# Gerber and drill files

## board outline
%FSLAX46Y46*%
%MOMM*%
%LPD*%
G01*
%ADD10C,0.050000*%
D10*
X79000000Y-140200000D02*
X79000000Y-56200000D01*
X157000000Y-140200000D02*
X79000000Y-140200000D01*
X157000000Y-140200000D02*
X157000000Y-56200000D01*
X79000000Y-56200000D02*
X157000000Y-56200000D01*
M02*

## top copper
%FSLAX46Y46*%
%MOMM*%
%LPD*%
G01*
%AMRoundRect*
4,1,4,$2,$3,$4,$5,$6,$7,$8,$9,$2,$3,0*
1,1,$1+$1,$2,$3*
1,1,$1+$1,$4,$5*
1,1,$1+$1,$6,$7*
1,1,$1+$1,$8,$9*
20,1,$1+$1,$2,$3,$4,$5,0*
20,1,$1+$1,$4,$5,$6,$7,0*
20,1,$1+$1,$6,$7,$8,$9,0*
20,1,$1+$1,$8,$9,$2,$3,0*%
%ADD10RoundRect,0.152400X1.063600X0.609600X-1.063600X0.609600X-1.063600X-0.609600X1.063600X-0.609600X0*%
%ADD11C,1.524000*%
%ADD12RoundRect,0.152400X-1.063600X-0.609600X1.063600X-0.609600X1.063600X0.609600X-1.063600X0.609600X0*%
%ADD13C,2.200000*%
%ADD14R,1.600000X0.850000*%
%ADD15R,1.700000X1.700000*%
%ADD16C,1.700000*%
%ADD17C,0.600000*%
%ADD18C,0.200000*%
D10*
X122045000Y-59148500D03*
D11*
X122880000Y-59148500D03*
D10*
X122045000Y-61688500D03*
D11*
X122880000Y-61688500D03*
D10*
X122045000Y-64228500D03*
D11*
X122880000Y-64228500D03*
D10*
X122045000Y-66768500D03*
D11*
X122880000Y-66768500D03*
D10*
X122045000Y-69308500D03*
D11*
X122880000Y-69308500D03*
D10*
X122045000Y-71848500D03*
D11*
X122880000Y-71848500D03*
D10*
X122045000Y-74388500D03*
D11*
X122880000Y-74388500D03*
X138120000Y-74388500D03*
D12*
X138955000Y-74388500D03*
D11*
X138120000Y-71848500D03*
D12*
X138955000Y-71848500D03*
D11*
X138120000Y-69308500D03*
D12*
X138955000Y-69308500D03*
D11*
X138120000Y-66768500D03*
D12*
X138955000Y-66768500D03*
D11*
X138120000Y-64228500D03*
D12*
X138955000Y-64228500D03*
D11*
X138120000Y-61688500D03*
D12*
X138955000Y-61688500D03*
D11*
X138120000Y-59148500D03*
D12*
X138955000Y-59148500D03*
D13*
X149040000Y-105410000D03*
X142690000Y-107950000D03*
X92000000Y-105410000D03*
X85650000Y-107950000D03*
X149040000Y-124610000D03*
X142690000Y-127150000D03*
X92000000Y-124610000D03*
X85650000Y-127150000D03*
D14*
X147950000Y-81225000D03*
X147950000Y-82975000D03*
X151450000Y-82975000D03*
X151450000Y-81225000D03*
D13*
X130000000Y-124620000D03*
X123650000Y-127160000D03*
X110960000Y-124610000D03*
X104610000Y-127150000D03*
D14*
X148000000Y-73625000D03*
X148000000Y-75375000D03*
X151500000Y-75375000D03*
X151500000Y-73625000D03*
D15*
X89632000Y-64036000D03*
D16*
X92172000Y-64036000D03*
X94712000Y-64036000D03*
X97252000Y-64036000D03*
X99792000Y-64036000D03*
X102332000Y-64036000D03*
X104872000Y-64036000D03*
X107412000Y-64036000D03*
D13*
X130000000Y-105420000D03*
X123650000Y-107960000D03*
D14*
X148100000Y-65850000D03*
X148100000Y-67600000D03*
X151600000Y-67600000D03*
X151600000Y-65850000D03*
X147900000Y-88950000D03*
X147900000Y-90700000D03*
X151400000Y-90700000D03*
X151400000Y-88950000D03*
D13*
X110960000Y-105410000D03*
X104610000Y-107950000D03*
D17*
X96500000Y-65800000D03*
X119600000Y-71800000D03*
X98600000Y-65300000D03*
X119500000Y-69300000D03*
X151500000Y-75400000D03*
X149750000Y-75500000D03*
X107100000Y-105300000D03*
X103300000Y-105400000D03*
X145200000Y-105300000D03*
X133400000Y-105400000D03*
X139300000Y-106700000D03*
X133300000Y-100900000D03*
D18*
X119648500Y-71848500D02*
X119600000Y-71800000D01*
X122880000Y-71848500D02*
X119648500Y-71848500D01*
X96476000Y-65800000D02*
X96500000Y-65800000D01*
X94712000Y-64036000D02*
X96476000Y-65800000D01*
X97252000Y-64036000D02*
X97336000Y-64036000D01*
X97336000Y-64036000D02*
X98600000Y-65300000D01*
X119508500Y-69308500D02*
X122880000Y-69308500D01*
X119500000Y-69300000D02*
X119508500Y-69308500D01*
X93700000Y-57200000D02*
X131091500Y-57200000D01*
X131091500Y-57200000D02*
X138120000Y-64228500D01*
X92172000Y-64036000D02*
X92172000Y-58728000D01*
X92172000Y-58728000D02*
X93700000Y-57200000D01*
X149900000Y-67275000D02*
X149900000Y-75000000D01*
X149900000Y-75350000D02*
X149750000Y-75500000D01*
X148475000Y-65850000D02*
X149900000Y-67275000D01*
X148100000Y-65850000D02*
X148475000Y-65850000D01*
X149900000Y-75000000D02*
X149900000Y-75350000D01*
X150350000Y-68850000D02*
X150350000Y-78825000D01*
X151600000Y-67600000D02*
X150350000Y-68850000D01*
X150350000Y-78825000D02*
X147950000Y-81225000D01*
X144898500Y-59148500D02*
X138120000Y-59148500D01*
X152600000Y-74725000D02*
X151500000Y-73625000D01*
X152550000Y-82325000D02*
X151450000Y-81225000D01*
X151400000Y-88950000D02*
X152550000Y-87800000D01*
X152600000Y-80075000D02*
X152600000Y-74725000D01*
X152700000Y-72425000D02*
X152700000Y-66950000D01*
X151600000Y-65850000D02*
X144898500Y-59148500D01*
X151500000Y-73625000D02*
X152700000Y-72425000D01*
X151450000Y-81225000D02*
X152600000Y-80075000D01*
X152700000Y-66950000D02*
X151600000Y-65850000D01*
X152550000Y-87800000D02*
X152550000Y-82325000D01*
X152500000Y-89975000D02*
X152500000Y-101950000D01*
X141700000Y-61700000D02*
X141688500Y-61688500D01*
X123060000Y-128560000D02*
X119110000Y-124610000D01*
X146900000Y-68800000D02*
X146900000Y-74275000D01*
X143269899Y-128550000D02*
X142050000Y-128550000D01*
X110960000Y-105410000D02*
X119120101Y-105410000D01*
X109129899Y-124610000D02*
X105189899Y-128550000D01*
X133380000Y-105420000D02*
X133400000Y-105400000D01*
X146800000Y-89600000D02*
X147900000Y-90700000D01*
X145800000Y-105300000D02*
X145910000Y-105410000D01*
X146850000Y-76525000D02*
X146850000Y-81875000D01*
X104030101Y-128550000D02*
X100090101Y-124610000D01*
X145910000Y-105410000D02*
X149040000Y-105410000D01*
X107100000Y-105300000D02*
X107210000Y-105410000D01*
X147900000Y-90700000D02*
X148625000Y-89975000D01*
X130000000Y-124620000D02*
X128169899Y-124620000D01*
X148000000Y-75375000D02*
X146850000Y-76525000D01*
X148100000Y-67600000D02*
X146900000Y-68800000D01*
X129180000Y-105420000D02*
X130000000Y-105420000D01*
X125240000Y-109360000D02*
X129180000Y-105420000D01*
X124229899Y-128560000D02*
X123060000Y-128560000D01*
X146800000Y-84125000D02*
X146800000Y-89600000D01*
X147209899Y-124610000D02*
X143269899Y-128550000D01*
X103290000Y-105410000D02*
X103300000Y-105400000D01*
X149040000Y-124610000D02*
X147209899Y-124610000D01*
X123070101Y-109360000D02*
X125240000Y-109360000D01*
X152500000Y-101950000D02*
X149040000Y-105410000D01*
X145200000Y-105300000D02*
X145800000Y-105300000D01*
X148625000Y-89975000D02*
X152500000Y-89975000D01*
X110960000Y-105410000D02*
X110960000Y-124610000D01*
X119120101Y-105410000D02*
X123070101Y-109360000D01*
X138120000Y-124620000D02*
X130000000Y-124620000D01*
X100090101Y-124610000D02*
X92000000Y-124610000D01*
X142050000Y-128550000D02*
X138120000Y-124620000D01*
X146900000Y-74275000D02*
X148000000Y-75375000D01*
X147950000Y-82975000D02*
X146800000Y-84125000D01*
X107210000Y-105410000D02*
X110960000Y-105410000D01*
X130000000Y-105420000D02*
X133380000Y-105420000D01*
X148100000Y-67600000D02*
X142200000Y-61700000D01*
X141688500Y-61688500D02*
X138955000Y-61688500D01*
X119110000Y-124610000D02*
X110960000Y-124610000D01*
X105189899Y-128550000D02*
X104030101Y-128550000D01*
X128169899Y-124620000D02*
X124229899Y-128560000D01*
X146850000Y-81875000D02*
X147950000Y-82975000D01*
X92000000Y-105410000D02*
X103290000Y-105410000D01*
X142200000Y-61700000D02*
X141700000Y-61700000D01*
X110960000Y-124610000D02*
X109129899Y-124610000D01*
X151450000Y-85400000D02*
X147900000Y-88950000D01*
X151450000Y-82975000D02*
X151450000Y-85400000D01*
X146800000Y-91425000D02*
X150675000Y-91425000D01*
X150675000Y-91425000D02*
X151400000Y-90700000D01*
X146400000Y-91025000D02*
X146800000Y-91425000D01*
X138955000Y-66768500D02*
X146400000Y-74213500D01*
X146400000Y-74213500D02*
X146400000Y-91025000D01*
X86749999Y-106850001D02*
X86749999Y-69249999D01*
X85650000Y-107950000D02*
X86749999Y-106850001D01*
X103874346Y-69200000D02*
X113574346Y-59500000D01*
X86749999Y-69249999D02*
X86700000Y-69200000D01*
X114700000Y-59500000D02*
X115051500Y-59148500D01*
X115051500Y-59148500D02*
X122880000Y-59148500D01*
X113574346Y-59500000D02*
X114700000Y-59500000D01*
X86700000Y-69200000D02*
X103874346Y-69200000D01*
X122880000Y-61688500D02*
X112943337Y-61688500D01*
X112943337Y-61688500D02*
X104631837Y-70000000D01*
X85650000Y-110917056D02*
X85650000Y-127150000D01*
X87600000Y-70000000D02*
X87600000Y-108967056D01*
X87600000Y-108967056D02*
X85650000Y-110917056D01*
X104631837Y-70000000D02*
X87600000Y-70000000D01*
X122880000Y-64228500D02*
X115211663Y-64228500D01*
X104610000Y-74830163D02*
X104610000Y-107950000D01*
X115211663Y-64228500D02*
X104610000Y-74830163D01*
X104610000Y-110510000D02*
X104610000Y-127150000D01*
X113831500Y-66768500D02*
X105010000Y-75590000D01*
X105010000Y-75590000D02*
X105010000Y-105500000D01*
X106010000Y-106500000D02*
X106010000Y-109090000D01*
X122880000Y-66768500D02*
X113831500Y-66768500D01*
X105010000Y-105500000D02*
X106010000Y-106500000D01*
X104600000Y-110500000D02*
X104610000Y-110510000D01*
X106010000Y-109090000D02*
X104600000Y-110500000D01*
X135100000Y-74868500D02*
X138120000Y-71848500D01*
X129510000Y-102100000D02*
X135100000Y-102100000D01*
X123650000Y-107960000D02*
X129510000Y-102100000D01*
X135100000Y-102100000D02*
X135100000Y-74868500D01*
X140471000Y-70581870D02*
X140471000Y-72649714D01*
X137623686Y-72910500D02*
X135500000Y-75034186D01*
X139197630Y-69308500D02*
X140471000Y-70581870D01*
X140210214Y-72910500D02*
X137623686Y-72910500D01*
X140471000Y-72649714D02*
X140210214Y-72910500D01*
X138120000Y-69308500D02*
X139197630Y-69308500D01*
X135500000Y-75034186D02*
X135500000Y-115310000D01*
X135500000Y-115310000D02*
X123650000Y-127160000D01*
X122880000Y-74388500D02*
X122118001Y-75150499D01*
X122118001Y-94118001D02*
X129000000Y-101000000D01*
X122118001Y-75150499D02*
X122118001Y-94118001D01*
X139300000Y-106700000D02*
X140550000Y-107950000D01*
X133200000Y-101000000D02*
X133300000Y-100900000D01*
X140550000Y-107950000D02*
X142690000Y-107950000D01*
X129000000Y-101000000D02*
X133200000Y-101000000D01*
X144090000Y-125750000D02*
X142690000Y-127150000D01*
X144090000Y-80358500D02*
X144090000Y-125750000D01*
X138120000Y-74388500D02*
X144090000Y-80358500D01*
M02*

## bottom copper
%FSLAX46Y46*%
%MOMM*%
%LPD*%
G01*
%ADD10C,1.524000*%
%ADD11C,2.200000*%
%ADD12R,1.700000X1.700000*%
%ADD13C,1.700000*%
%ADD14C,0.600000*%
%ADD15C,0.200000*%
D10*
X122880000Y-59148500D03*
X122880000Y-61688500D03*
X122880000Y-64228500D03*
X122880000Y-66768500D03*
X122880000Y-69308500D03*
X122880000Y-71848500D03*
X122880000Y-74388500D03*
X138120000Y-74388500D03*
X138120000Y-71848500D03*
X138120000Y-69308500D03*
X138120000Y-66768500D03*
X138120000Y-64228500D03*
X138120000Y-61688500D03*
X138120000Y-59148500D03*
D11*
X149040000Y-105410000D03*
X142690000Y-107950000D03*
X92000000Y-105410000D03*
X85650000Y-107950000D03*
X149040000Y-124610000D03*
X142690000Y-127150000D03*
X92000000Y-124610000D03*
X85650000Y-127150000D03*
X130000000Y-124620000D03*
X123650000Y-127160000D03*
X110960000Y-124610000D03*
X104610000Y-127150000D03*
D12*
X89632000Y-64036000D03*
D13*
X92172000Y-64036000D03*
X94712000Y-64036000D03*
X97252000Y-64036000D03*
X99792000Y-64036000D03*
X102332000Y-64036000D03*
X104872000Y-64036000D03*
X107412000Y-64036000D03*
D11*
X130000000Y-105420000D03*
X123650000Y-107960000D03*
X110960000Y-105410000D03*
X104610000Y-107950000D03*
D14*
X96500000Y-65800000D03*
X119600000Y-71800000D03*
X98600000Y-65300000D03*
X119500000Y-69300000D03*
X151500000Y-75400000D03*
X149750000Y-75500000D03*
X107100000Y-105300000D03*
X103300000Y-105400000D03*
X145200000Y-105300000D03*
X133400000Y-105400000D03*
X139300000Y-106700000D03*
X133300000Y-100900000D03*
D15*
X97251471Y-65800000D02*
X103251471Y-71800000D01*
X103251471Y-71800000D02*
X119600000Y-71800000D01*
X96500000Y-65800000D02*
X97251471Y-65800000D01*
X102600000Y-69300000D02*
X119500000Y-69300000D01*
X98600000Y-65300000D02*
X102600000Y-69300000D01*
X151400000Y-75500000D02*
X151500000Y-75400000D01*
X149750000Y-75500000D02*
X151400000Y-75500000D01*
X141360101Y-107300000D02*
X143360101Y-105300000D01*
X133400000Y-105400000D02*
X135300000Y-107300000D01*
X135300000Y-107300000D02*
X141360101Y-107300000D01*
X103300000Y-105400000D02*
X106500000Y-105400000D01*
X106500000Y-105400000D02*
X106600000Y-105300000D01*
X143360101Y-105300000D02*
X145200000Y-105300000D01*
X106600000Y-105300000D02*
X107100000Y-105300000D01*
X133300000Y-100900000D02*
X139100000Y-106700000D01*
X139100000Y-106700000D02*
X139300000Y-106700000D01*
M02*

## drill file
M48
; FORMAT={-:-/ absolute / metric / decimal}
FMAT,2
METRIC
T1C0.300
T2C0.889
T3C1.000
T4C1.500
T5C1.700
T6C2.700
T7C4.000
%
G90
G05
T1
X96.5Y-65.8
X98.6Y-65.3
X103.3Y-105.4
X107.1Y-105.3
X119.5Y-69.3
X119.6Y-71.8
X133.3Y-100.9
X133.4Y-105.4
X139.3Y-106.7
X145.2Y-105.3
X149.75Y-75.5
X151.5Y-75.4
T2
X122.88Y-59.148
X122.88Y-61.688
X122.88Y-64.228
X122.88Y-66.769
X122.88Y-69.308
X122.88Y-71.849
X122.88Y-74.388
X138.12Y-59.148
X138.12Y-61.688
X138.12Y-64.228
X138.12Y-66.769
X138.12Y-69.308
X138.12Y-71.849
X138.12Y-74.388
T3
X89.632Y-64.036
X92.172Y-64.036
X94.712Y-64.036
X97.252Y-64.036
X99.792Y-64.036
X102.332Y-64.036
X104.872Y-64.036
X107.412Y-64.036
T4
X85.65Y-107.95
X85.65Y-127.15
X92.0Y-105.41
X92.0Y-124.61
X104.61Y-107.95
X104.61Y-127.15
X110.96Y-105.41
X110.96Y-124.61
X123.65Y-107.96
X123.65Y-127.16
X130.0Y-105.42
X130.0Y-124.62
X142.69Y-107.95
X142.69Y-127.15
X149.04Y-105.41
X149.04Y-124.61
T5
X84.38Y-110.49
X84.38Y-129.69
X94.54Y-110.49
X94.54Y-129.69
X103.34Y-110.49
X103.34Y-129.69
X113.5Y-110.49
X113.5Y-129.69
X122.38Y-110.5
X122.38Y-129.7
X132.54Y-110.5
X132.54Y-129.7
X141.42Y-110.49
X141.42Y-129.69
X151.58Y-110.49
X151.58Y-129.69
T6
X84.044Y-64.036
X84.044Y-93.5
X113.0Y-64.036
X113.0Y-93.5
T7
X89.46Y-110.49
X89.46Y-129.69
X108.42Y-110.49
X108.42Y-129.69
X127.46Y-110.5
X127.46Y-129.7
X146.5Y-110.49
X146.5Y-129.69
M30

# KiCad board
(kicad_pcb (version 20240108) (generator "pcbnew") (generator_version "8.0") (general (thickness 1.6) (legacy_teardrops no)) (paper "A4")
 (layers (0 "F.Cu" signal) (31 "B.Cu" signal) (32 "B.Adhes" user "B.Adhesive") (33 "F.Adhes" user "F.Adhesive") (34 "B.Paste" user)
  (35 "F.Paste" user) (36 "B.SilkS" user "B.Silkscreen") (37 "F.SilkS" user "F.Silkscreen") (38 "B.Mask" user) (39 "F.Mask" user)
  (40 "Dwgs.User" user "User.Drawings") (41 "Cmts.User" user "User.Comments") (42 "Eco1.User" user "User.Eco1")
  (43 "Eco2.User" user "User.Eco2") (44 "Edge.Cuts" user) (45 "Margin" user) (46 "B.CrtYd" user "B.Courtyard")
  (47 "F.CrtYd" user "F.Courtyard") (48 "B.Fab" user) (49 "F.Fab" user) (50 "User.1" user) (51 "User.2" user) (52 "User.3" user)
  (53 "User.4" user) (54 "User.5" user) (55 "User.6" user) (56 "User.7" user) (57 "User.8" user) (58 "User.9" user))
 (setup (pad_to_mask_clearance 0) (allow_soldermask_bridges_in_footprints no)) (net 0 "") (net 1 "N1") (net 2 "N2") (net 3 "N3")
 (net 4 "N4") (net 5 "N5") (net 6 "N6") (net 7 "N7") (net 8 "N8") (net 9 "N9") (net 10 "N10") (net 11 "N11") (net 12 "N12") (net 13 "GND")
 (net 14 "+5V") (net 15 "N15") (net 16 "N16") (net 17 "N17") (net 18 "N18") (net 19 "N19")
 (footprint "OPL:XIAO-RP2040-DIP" (layer "F.Cu") (at 130.5 66.7685)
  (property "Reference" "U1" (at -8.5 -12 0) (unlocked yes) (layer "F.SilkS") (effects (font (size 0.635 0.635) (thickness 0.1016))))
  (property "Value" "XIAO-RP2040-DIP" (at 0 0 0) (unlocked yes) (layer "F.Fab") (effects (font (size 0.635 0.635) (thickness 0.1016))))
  (pad "1" smd roundrect (at -8.455 -7.62 180) (size 2.432 1.524) (layers "F.Cu" "F.Mask") (roundrect_rratio 0.1) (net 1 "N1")
   (thermal_bridge_angle 45))
  (pad "1" thru_hole circle (at -7.62 -7.62 180) (size 1.524 1.524) (drill 0.889) (layers "*.Cu" "*.Mask") (remove_unused_layers no)
   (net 1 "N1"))
  (pad "2" smd roundrect (at -8.455 -5.08 180) (size 2.432 1.524) (layers "F.Cu" "F.Mask") (roundrect_rratio 0.1) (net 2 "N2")
   (thermal_bridge_angle 45))
  (pad "2" thru_hole circle (at -7.62 -5.08 180) (size 1.524 1.524) (drill 0.889) (layers "*.Cu" "*.Mask") (remove_unused_layers no)
   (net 2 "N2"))
  (pad "3" smd roundrect (at -8.455 -2.54 180) (size 2.432 1.524) (layers "F.Cu" "F.Mask") (roundrect_rratio 0.1) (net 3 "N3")
   (thermal_bridge_angle 45))
  (pad "3" thru_hole circle (at -7.62 -2.54 180) (size 1.524 1.524) (drill 0.889) (layers "*.Cu" "*.Mask") (remove_unused_layers no)
   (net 3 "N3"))
  (pad "4" smd roundrect (at -8.455 0 180) (size 2.432 1.524) (layers "F.Cu" "F.Mask") (roundrect_rratio 0.1) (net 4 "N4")
   (thermal_bridge_angle 45))
  (pad "4" thru_hole circle (at -7.62 0 180) (size 1.524 1.524) (drill 0.889) (layers "*.Cu" "*.Mask") (remove_unused_layers no)
   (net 4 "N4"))
  (pad "5" smd roundrect (at -8.455 2.54 180) (size 2.432 1.524) (layers "F.Cu" "F.Mask") (roundrect_rratio 0.1) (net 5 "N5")
   (thermal_bridge_angle 45))
  (pad "5" thru_hole circle (at -7.62 2.54 180) (size 1.524 1.524) (drill 0.889) (layers "*.Cu" "*.Mask") (remove_unused_layers no)
   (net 5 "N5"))
  (pad "6" smd roundrect (at -8.455 5.08 180) (size 2.432 1.524) (layers "F.Cu" "F.Mask") (roundrect_rratio 0.1) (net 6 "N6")
   (thermal_bridge_angle 45))
  (pad "6" thru_hole circle (at -7.62 5.08 180) (size 1.524 1.524) (drill 0.889) (layers "*.Cu" "*.Mask") (remove_unused_layers no)
   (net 6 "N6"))
  (pad "7" smd roundrect (at -8.455 7.62 180) (size 2.432 1.524) (layers "F.Cu" "F.Mask") (roundrect_rratio 0.1) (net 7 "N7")
   (thermal_bridge_angle 45))
  (pad "7" thru_hole circle (at -7.62 7.62 180) (size 1.524 1.524) (drill 0.889) (layers "*.Cu" "*.Mask") (remove_unused_layers no)
   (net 7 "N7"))
  (pad "8" thru_hole circle (at 7.62 7.62) (size 1.524 1.524) (drill 0.889) (layers "*.Cu" "*.Mask") (remove_unused_layers no) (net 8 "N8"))
  (pad "8" smd roundrect (at 8.455 7.62) (size 2.432 1.524) (layers "F.Cu" "F.Mask") (roundrect_rratio 0.1) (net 8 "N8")
   (thermal_bridge_angle 45))
  (pad "9" thru_hole circle (at 7.62 5.08) (size 1.524 1.524) (drill 0.889) (layers "*.Cu" "*.Mask") (remove_unused_layers no) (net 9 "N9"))
  (pad "9" smd roundrect (at 8.455 5.08) (size 2.432 1.524) (layers "F.Cu" "F.Mask") (roundrect_rratio 0.1) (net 9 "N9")
   (thermal_bridge_angle 45))
  (pad "10" thru_hole circle (at 7.62 2.54) (size 1.524 1.524) (drill 0.889) (layers "*.Cu" "*.Mask") (remove_unused_layers no)
   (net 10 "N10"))
  (pad "10" smd roundrect (at 8.455 2.54) (size 2.432 1.524) (layers "F.Cu" "F.Mask") (roundrect_rratio 0.1) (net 10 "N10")
   (thermal_bridge_angle 45))
  (pad "11" thru_hole circle (at 7.62 0) (size 1.524 1.524) (drill 0.889) (layers "*.Cu" "*.Mask") (remove_unused_layers no) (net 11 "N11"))
  (pad "11" smd roundrect (at 8.455 0) (size 2.432 1.524) (layers "F.Cu" "F.Mask") (roundrect_rratio 0.1) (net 11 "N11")
   (thermal_bridge_angle 45))
  (pad "12" thru_hole circle (at 7.62 -2.54) (size 1.524 1.524) (drill 0.889) (layers "*.Cu" "*.Mask") (remove_unused_layers no)
   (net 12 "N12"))
  (pad "12" smd roundrect (at 8.455 -2.54) (size 2.432 1.524) (layers "F.Cu" "F.Mask") (roundrect_rratio 0.1) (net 12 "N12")
   (thermal_bridge_angle 45))
  (pad "13" thru_hole circle (at 7.62 -5.08) (size 1.524 1.524) (drill 0.889) (layers "*.Cu" "*.Mask") (remove_unused_layers no)
   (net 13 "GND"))
  (pad "13" smd roundrect (at 8.455 -5.08) (size 2.432 1.524) (layers "F.Cu" "F.Mask") (roundrect_rratio 0.1) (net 13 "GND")
   (thermal_bridge_angle 45))
  (pad "14" thru_hole circle (at 7.62 -7.62) (size 1.524 1.524) (drill 0.889) (layers "*.Cu" "*.Mask") (remove_unused_layers no)
   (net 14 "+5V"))
  (pad "14" smd roundrect (at 8.455 -7.62) (size 2.432 1.524) (layers "F.Cu" "F.Mask") (roundrect_rratio 0.1) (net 14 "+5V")
   (thermal_bridge_angle 45)))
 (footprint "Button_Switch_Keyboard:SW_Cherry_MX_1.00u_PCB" (layer "F.Cu") (at 149.04 105.41)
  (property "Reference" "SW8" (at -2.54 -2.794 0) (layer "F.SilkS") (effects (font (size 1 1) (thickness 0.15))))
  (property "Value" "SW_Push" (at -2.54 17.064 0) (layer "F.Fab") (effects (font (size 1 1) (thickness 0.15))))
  (pad "" np_thru_hole circle (at -7.62 5.08) (size 1.7 1.7) (drill 1.7) (layers "*.Cu" "*.Mask"))
  (pad "" np_thru_hole circle (at -2.54 5.08) (size 4 4) (drill 4) (layers "*.Cu" "*.Mask"))
  (pad "" np_thru_hole circle (at 2.54 5.08) (size 1.7 1.7) (drill 1.7) (layers "*.Cu" "*.Mask"))
  (pad "1" thru_hole circle (at 0 0) (size 2.2 2.2) (drill 1.5) (layers "*.Cu" "*.Mask") (remove_unused_layers no) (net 13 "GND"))
  (pad "2" thru_hole circle (at -6.35 2.54) (size 2.2 2.2) (drill 1.5) (layers "*.Cu" "*.Mask") (remove_unused_layers no) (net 7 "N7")))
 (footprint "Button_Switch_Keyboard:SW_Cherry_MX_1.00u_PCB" (layer "F.Cu") (at 92 105.41)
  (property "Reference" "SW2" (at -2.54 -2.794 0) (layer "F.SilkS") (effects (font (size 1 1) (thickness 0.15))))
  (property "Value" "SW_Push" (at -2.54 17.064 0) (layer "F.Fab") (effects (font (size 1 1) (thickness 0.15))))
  (pad "" np_thru_hole circle (at -7.62 5.08) (size 1.7 1.7) (drill 1.7) (layers "*.Cu" "*.Mask"))
  (pad "" np_thru_hole circle (at -2.54 5.08) (size 4 4) (drill 4) (layers "*.Cu" "*.Mask"))
  (pad "" np_thru_hole circle (at 2.54 5.08) (size 1.7 1.7) (drill 1.7) (layers "*.Cu" "*.Mask"))
  (pad "1" thru_hole circle (at 0 0) (size 2.2 2.2) (drill 1.5) (layers "*.Cu" "*.Mask") (remove_unused_layers no) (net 13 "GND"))
  (pad "2" thru_hole circle (at -6.35 2.54) (size 2.2 2.2) (drill 1.5) (layers "*.Cu" "*.Mask") (remove_unused_layers no) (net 1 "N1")))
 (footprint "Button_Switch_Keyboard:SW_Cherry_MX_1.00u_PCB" (layer "F.Cu") (at 149.04 124.61)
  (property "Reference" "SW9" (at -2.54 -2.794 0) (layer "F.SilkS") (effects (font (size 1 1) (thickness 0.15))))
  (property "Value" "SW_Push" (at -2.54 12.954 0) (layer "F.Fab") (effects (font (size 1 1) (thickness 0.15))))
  (pad "" np_thru_hole circle (at -7.62 5.08) (size 1.7 1.7) (drill 1.7) (layers "*.Cu" "*.Mask"))
  (pad "" np_thru_hole circle (at -2.54 5.08) (size 4 4) (drill 4) (layers "*.Cu" "*.Mask"))
  (pad "" np_thru_hole circle (at 2.54 5.08) (size 1.7 1.7) (drill 1.7) (layers "*.Cu" "*.Mask"))
  (pad "1" thru_hole circle (at 0 0) (size 2.2 2.2) (drill 1.5) (layers "*.Cu" "*.Mask") (remove_unused_layers no) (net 13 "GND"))
  (pad "2" thru_hole circle (at -6.35 2.54) (size 2.2 2.2) (drill 1.5) (layers "*.Cu" "*.Mask") (remove_unused_layers no) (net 8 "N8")))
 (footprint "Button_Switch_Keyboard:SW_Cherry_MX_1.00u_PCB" (layer "F.Cu") (at 92 124.61)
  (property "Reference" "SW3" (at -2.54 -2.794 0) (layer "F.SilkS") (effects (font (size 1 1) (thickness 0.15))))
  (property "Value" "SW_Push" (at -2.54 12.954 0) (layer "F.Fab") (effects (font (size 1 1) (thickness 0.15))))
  (pad "" np_thru_hole circle (at -7.62 5.08) (size 1.7 1.7) (drill 1.7) (layers "*.Cu" "*.Mask"))
  (pad "" np_thru_hole circle (at -2.54 5.08) (size 4 4) (drill 4) (layers "*.Cu" "*.Mask"))
  (pad "" np_thru_hole circle (at 2.54 5.08) (size 1.7 1.7) (drill 1.7) (layers "*.Cu" "*.Mask"))
  (pad "1" thru_hole circle (at 0 0) (size 2.2 2.2) (drill 1.5) (layers "*.Cu" "*.Mask") (remove_unused_layers no) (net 13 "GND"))
  (pad "2" thru_hole circle (at -6.35 2.54) (size 2.2 2.2) (drill 1.5) (layers "*.Cu" "*.Mask") (remove_unused_layers no) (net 2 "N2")))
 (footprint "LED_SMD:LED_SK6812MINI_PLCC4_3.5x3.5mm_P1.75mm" (layer "F.Cu") (at 149.7 82.1)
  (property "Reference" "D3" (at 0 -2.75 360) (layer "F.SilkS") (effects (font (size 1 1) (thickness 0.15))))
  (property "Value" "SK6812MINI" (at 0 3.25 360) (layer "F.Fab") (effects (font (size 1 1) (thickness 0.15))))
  (pad "1" smd rect (at -1.75 -0.875) (size 1.6 0.85) (layers "F.Cu" "F.Paste" "F.Mask") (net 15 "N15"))
  (pad "2" smd rect (at -1.75 0.875) (size 1.6 0.85) (layers "F.Cu" "F.Paste" "F.Mask") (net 13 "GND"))
  (pad "3" smd rect (at 1.75 0.875) (size 1.6 0.85) (layers "F.Cu" "F.Paste" "F.Mask") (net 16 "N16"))
  (pad "4" smd rect (at 1.75 -0.875) (size 1.6 0.85) (layers "F.Cu" "F.Paste" "F.Mask") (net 14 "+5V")))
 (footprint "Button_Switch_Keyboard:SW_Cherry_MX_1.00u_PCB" (layer "F.Cu") (at 130 124.62)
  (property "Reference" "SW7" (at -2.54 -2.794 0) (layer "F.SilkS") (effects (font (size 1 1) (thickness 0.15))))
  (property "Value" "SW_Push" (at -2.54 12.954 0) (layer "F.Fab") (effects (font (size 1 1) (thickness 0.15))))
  (pad "" np_thru_hole circle (at -7.62 5.08) (size 1.7 1.7) (drill 1.7) (layers "*.Cu" "*.Mask"))
  (pad "" np_thru_hole circle (at -2.54 5.08) (size 4 4) (drill 4) (layers "*.Cu" "*.Mask"))
  (pad "" np_thru_hole circle (at 2.54 5.08) (size 1.7 1.7) (drill 1.7) (layers "*.Cu" "*.Mask"))
  (pad "1" thru_hole circle (at 0 0) (size 2.2 2.2) (drill 1.5) (layers "*.Cu" "*.Mask") (remove_unused_layers no) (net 13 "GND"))
  (pad "2" thru_hole circle (at -6.35 2.54) (size 2.2 2.2) (drill 1.5) (layers "*.Cu" "*.Mask") (remove_unused_layers no) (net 10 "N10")))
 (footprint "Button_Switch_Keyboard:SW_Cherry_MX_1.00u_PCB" (layer "F.Cu") (at 110.96 124.61)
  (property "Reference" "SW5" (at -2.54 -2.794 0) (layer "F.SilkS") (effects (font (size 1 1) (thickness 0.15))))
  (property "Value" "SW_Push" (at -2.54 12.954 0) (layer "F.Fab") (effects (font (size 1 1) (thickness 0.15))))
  (pad "" np_thru_hole circle (at -7.62 5.08) (size 1.7 1.7) (drill 1.7) (layers "*.Cu" "*.Mask"))
  (pad "" np_thru_hole circle (at -2.54 5.08) (size 4 4) (drill 4) (layers "*.Cu" "*.Mask"))
  (pad "" np_thru_hole circle (at 2.54 5.08) (size 1.7 1.7) (drill 1.7) (layers "*.Cu" "*.Mask"))
  (pad "1" thru_hole circle (at 0 0) (size 2.2 2.2) (drill 1.5) (layers "*.Cu" "*.Mask") (remove_unused_layers no) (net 13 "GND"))
  (pad "2" thru_hole circle (at -6.35 2.54) (size 2.2 2.2) (drill 1.5) (layers "*.Cu" "*.Mask") (remove_unused_layers no) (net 4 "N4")))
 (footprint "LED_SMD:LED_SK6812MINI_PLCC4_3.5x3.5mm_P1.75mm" (layer "F.Cu") (at 149.75 74.5)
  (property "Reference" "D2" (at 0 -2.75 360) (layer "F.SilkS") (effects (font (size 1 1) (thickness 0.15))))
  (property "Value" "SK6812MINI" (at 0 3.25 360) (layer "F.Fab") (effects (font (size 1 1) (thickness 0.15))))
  (pad "1" smd rect (at -1.75 -0.875) (size 1.6 0.85) (layers "F.Cu" "F.Paste" "F.Mask") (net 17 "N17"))
  (pad "2" smd rect (at -1.75 0.875) (size 1.6 0.85) (layers "F.Cu" "F.Paste" "F.Mask") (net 13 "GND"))
  (pad "3" smd rect (at 1.75 0.875) (size 1.6 0.85) (layers "F.Cu" "F.Paste" "F.Mask") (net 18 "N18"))
  (pad "4" smd rect (at 1.75 -0.875) (size 1.6 0.85) (layers "F.Cu" "F.Paste" "F.Mask") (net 14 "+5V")))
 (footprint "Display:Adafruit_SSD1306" (layer "F.Cu") (at 89.632 64.036)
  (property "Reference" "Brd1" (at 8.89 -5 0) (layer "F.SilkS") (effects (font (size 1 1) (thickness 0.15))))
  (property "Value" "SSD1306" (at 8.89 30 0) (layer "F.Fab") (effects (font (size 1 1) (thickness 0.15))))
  (pad "" np_thru_hole circle (at -5.588 0) (size 2.7 2.7) (drill 2.7) (layers "*.Cu" "*.Mask"))
  (pad "" np_thru_hole circle (at -5.588 29.464) (size 2.7 2.7) (drill 2.7) (layers "*.Cu" "*.Mask"))
  (pad "" np_thru_hole circle (at 23.368 0) (size 2.7 2.7) (drill 2.7) (layers "*.Cu" "*.Mask"))
  (pad "" np_thru_hole circle (at 23.368 29.464) (size 2.7 2.7) (drill 2.7) (layers "*.Cu" "*.Mask"))
  (pad "1" thru_hole rect (at 0 0) (size 1.7 1.7) (drill 1) (layers "*.Cu" "*.Mask") (remove_unused_layers no) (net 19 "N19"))
  (pad "2" thru_hole circle (at 2.54 0) (size 1.7 1.7) (drill 1) (layers "*.Cu" "*.Mask") (remove_unused_layers no) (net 12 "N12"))
  (pad "3" thru_hole circle (at 5.08 0) (size 1.7 1.7) (drill 1) (layers "*.Cu" "*.Mask") (remove_unused_layers no) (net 6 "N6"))
  (pad "4" thru_hole circle (at 7.62 0) (size 1.7 1.7) (drill 1) (layers "*.Cu" "*.Mask") (remove_unused_layers no) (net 5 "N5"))
  (pad "5" thru_hole circle (at 10.16 0) (size 1.7 1.7) (drill 1) (layers "*.Cu" "*.Mask") (remove_unused_layers no))
  (pad "6" thru_hole circle (at 12.7 0) (size 1.7 1.7) (drill 1) (layers "*.Cu" "*.Mask") (remove_unused_layers no))
  (pad "7" thru_hole circle (at 15.24 0) (size 1.7 1.7) (drill 1) (layers "*.Cu" "*.Mask") (remove_unused_layers no))
  (pad "8" thru_hole circle (at 17.78 0) (size 1.7 1.7) (drill 1) (layers "*.Cu" "*.Mask") (remove_unused_layers no)))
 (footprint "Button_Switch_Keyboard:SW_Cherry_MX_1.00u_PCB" (layer "F.Cu") (at 130 105.42)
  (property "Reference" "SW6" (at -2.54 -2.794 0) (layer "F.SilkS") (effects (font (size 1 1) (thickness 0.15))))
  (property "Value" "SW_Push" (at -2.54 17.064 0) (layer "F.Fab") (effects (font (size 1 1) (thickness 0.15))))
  (pad "" np_thru_hole circle (at -7.62 5.08) (size 1.7 1.7) (drill 1.7) (layers "*.Cu" "*.Mask"))
  (pad "" np_thru_hole circle (at -2.54 5.08) (size 4 4) (drill 4) (layers "*.Cu" "*.Mask"))
  (pad "" np_thru_hole circle (at 2.54 5.08) (size 1.7 1.7) (drill 1.7) (layers "*.Cu" "*.Mask"))
  (pad "1" thru_hole circle (at 0 0) (size 2.2 2.2) (drill 1.5) (layers "*.Cu" "*.Mask") (remove_unused_layers no) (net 13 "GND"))
  (pad "2" thru_hole circle (at -6.35 2.54) (size 2.2 2.2) (drill 1.5) (layers "*.Cu" "*.Mask") (remove_unused_layers no) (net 9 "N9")))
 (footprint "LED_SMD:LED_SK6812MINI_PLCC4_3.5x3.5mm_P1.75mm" (layer "F.Cu") (at 149.85 66.725)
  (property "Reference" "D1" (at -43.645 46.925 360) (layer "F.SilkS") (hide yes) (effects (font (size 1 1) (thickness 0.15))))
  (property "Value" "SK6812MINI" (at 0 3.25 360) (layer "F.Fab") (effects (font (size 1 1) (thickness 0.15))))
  (pad "1" smd rect (at -1.75 -0.875) (size 1.6 0.85) (layers "F.Cu" "F.Paste" "F.Mask") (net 18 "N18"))
  (pad "2" smd rect (at -1.75 0.875) (size 1.6 0.85) (layers "F.Cu" "F.Paste" "F.Mask") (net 13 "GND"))
  (pad "3" smd rect (at 1.75 0.875) (size 1.6 0.85) (layers "F.Cu" "F.Paste" "F.Mask") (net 15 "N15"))
  (pad "4" smd rect (at 1.75 -0.875) (size 1.6 0.85) (layers "F.Cu" "F.Paste" "F.Mask") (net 14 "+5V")))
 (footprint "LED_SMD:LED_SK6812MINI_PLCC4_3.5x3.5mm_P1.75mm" (layer "F.Cu") (at 149.65 89.825)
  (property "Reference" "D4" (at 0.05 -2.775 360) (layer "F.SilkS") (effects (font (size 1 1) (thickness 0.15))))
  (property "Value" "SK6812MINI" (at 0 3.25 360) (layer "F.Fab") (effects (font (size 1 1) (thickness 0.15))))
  (pad "1" smd rect (at -1.75 -0.875) (size 1.6 0.85) (layers "F.Cu" "F.Paste" "F.Mask") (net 16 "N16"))
  (pad "2" smd rect (at -1.75 0.875) (size 1.6 0.85) (layers "F.Cu" "F.Paste" "F.Mask") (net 13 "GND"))
  (pad "3" smd rect (at 1.75 0.875) (size 1.6 0.85) (layers "F.Cu" "F.Paste" "F.Mask") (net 11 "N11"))
  (pad "4" smd rect (at 1.75 -0.875) (size 1.6 0.85) (layers "F.Cu" "F.Paste" "F.Mask") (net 14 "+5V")))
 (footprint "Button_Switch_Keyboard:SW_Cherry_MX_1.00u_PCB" (layer "F.Cu") (at 110.96 105.41)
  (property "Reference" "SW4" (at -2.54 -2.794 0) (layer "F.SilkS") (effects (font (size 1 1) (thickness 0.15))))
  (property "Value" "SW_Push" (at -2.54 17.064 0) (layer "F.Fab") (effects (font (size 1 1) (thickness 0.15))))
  (pad "" np_thru_hole circle (at -7.62 5.08) (size 1.7 1.7) (drill 1.7) (layers "*.Cu" "*.Mask"))
  (pad "" np_thru_hole circle (at -2.54 5.08) (size 4 4) (drill 4) (layers "*.Cu" "*.Mask"))
  (pad "" np_thru_hole circle (at 2.54 5.08) (size 1.7 1.7) (drill 1.7) (layers "*.Cu" "*.Mask"))
  (pad "1" thru_hole circle (at 0 0) (size 2.2 2.2) (drill 1.5) (layers "*.Cu" "*.Mask") (remove_unused_layers no) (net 13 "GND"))
  (pad "2" thru_hole circle (at -6.35 2.54) (size 2.2 2.2) (drill 1.5) (layers "*.Cu" "*.Mask") (remove_unused_layers no) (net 3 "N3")))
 (gr_line (start 79 140.2) (end 79 56.2) (stroke (width 0.05) (type default)) (layer "Edge.Cuts"))
 (gr_line (start 157 140.2) (end 79 140.2) (stroke (width 0.05) (type default)) (layer "Edge.Cuts"))
 (gr_line (start 157 140.2) (end 157 56.2) (stroke (width 0.05) (type default)) (layer "Edge.Cuts"))
 (gr_line (start 79 56.2) (end 157 56.2) (stroke (width 0.05) (type default)) (layer "Edge.Cuts"))
 (segment (start 119.6485 71.8485) (end 119.6 71.8) (width 0.2) (layer "F.Cu") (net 6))
 (segment (start 122.88 71.8485) (end 119.6485 71.8485) (width 0.2) (layer "F.Cu") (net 6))
 (segment (start 96.476 65.8) (end 96.5 65.8) (width 0.2) (layer "F.Cu") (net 6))
 (segment (start 94.712 64.036) (end 96.476 65.8) (width 0.2) (layer "F.Cu") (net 6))
 (via (at 96.5 65.8) (size 0.6) (drill 0.3) (layers "F.Cu" "B.Cu") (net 6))
 (via (at 119.6 71.8) (size 0.6) (drill 0.3) (layers "F.Cu" "B.Cu") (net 6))
 (segment (start 97.251471 65.8) (end 103.251471 71.8) (width 0.2) (layer "B.Cu") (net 6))
 (segment (start 103.251471 71.8) (end 119.6 71.8) (width 0.2) (layer "B.Cu") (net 6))
 (segment (start 96.5 65.8) (end 97.251471 65.8) (width 0.2) (layer "B.Cu") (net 6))
 (segment (start 97.252 64.036) (end 97.336 64.036) (width 0.2) (layer "F.Cu") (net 5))
 (segment (start 97.336 64.036) (end 98.6 65.3) (width 0.2) (layer "F.Cu") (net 5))
 (segment (start 119.5085 69.3085) (end 122.88 69.3085) (width 0.2) (layer "F.Cu") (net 5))
 (segment (start 119.5 69.3) (end 119.5085 69.3085) (width 0.2) (layer "F.Cu") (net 5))
 (via (at 98.6 65.3) (size 0.6) (drill 0.3) (layers "F.Cu" "B.Cu") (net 5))
 (via (at 119.5 69.3) (size 0.6) (drill 0.3) (layers "F.Cu" "B.Cu") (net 5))
 (segment (start 102.6 69.3) (end 119.5 69.3) (width 0.2) (layer "B.Cu") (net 5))
 (segment (start 98.6 65.3) (end 102.6 69.3) (width 0.2) (layer "B.Cu") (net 5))
 (segment (start 93.7 57.2) (end 131.0915 57.2) (width 0.2) (layer "F.Cu") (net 12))
 (segment (start 131.0915 57.2) (end 138.12 64.2285) (width 0.2) (layer "F.Cu") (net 12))
 (segment (start 92.172 64.036) (end 92.172 58.728) (width 0.2) (layer "F.Cu") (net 12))
 (segment (start 92.172 58.728) (end 93.7 57.2) (width 0.2) (layer "F.Cu") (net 12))
 (segment (start 149.9 67.275) (end 149.9 75) (width 0.2) (layer "F.Cu") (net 18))
 (segment (start 149.9 75.35) (end 149.75 75.5) (width 0.2) (layer "F.Cu") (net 18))
 (segment (start 148.475 65.85) (end 149.9 67.275) (width 0.2) (layer "F.Cu") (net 18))
 (segment (start 148.1 65.85) (end 148.475 65.85) (width 0.2) (layer "F.Cu") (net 18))
 (segment (start 149.9 75) (end 149.9 75.35) (width 0.2) (layer "F.Cu") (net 18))
 (via (at 151.5 75.4) (size 0.6) (drill 0.3) (layers "F.Cu" "B.Cu") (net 18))
 (via (at 149.75 75.5) (size 0.6) (drill 0.3) (layers "F.Cu" "B.Cu") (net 18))
 (segment (start 151.4 75.5) (end 151.5 75.4) (width 0.2) (layer "B.Cu") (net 18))
 (segment (start 149.75 75.5) (end 151.4 75.5) (width 0.2) (layer "B.Cu") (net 18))
 (segment (start 150.35 68.85) (end 150.35 78.825) (width 0.2) (layer "F.Cu") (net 15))
 (segment (start 151.6 67.6) (end 150.35 68.85) (width 0.2) (layer "F.Cu") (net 15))
 (segment (start 150.35 78.825) (end 147.95 81.225) (width 0.2) (layer "F.Cu") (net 15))
 (segment (start 144.8985 59.1485) (end 138.12 59.1485) (width 0.2) (layer "F.Cu") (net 14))
 (segment (start 152.6 74.725) (end 151.5 73.625) (width 0.2) (layer "F.Cu") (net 14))
 (segment (start 152.55 82.325) (end 151.45 81.225) (width 0.2) (layer "F.Cu") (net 14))
 (segment (start 151.4 88.95) (end 152.55 87.8) (width 0.2) (layer "F.Cu") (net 14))
 (segment (start 152.6 80.075) (end 152.6 74.725) (width 0.2) (layer "F.Cu") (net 14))
 (segment (start 152.7 72.425) (end 152.7 66.95) (width 0.2) (layer "F.Cu") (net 14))
 (segment (start 151.6 65.85) (end 144.8985 59.1485) (width 0.2) (layer "F.Cu") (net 14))
 (segment (start 151.5 73.625) (end 152.7 72.425) (width 0.2) (layer "F.Cu") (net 14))
 (segment (start 151.45 81.225) (end 152.6 80.075) (width 0.2) (layer "F.Cu") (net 14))
 (segment (start 152.7 66.95) (end 151.6 65.85) (width 0.2) (layer "F.Cu") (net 14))
 (segment (start 152.55 87.8) (end 152.55 82.325) (width 0.2) (layer "F.Cu") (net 14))
 (segment (start 152.5 89.975) (end 152.5 101.95) (width 0.2) (layer "F.Cu") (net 13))
 (segment (start 141.7 61.7) (end 141.6885 61.6885) (width 0.2) (layer "F.Cu") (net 13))
 (segment (start 123.06 128.56) (end 119.11 124.61) (width 0.2) (layer "F.Cu") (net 13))
 (segment (start 146.9 68.8) (end 146.9 74.275) (width 0.2) (layer "F.Cu") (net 13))
 (segment (start 143.269899 128.55) (end 142.05 128.55) (width 0.2) (layer "F.Cu") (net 13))
 (segment (start 110.96 105.41) (end 119.120101 105.41) (width 0.2) (layer "F.Cu") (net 13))
 (segment (start 109.129899 124.61) (end 105.189899 128.55) (width 0.2) (layer "F.Cu") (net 13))
 (segment (start 133.38 105.42) (end 133.4 105.4) (width 0.2) (layer "F.Cu") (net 13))
 (segment (start 146.8 89.6) (end 147.9 90.7) (width 0.2) (layer "F.Cu") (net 13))
 (segment (start 145.8 105.3) (end 145.91 105.41) (width 0.2) (layer "F.Cu") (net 13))
 (segment (start 146.85 76.525) (end 146.85 81.875) (width 0.2) (layer "F.Cu") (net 13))
 (segment (start 104.030101 128.55) (end 100.090101 124.61) (width 0.2) (layer "F.Cu") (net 13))
 (segment (start 145.91 105.41) (end 149.04 105.41) (width 0.2) (layer "F.Cu") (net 13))
 (segment (start 107.1 105.3) (end 107.21 105.41) (width 0.2) (layer "F.Cu") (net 13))
 (segment (start 147.9 90.7) (end 148.625 89.975) (width 0.2) (layer "F.Cu") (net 13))
 (segment (start 130 124.62) (end 128.169899 124.62) (width 0.2) (layer "F.Cu") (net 13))
 (segment (start 148 75.375) (end 146.85 76.525) (width 0.2) (layer "F.Cu") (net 13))
 (segment (start 148.1 67.6) (end 146.9 68.8) (width 0.2) (layer "F.Cu") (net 13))
 (segment (start 129.18 105.42) (end 130 105.42) (width 0.2) (layer "F.Cu") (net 13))
 (segment (start 125.24 109.36) (end 129.18 105.42) (width 0.2) (layer "F.Cu") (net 13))
 (segment (start 124.229899 128.56) (end 123.06 128.56) (width 0.2) (layer "F.Cu") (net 13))
 (segment (start 146.8 84.125) (end 146.8 89.6) (width 0.2) (layer "F.Cu") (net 13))
 (segment (start 147.209899 124.61) (end 143.269899 128.55) (width 0.2) (layer "F.Cu") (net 13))
 (segment (start 103.29 105.41) (end 103.3 105.4) (width 0.2) (layer "F.Cu") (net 13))
 (segment (start 149.04 124.61) (end 147.209899 124.61) (width 0.2) (layer "F.Cu") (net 13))
 (segment (start 123.070101 109.36) (end 125.24 109.36) (width 0.2) (layer "F.Cu") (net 13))
 (segment (start 152.5 101.95) (end 149.04 105.41) (width 0.2) (layer "F.Cu") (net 13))
 (segment (start 145.2 105.3) (end 145.8 105.3) (width 0.2) (layer "F.Cu") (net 13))
 (segment (start 148.625 89.975) (end 152.5 89.975) (width 0.2) (layer "F.Cu") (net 13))
 (segment (start 110.96 105.41) (end 110.96 124.61) (width 0.2) (layer "F.Cu") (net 13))
 (segment (start 119.120101 105.41) (end 123.070101 109.36) (width 0.2) (layer "F.Cu") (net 13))
 (segment (start 138.12 124.62) (end 130 124.62) (width 0.2) (layer "F.Cu") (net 13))
 (segment (start 100.090101 124.61) (end 92 124.61) (width 0.2) (layer "F.Cu") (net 13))
 (segment (start 142.05 128.55) (end 138.12 124.62) (width 0.2) (layer "F.Cu") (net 13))
 (segment (start 146.9 74.275) (end 148 75.375) (width 0.2) (layer "F.Cu") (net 13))
 (segment (start 147.95 82.975) (end 146.8 84.125) (width 0.2) (layer "F.Cu") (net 13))
 (segment (start 107.21 105.41) (end 110.96 105.41) (width 0.2) (layer "F.Cu") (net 13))
 (segment (start 130 105.42) (end 133.38 105.42) (width 0.2) (layer "F.Cu") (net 13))
 (segment (start 148.1 67.6) (end 142.2 61.7) (width 0.2) (layer "F.Cu") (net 13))
 (segment (start 141.6885 61.6885) (end 138.955 61.6885) (width 0.2) (layer "F.Cu") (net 13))
 (segment (start 119.11 124.61) (end 110.96 124.61) (width 0.2) (layer "F.Cu") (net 13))
 (segment (start 105.189899 128.55) (end 104.030101 128.55) (width 0.2) (layer "F.Cu") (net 13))
 (segment (start 128.169899 124.62) (end 124.229899 128.56) (width 0.2) (layer "F.Cu") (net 13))
 (segment (start 146.85 81.875) (end 147.95 82.975) (width 0.2) (layer "F.Cu") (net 13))
 (segment (start 92 105.41) (end 103.29 105.41) (width 0.2) (layer "F.Cu") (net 13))
 (segment (start 142.2 61.7) (end 141.7 61.7) (width 0.2) (layer "F.Cu") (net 13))
 (segment (start 110.96 124.61) (end 109.129899 124.61) (width 0.2) (layer "F.Cu") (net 13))
 (via (at 107.1 105.3) (size 0.6) (drill 0.3) (layers "F.Cu" "B.Cu") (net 13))
 (via (at 103.3 105.4) (size 0.6) (drill 0.3) (layers "F.Cu" "B.Cu") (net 13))
 (via (at 145.2 105.3) (size 0.6) (drill 0.3) (layers "F.Cu" "B.Cu") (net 13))
 (via (at 133.4 105.4) (size 0.6) (drill 0.3) (layers "F.Cu" "B.Cu") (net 13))
 (segment (start 141.360101 107.3) (end 143.360101 105.3) (width 0.2) (layer "B.Cu") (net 13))
 (segment (start 133.4 105.4) (end 135.3 107.3) (width 0.2) (layer "B.Cu") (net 13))
 (segment (start 135.3 107.3) (end 141.360101 107.3) (width 0.2) (layer "B.Cu") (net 13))
 (segment (start 103.3 105.4) (end 106.5 105.4) (width 0.2) (layer "B.Cu") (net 13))
 (segment (start 106.5 105.4) (end 106.6 105.3) (width 0.2) (layer "B.Cu") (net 13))
 (segment (start 143.360101 105.3) (end 145.2 105.3) (width 0.2) (layer "B.Cu") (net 13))
 (segment (start 106.6 105.3) (end 107.1 105.3) (width 0.2) (layer "B.Cu") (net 13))
 (segment (start 151.45 85.4) (end 147.9 88.95) (width 0.2) (layer "F.Cu") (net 16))
 (segment (start 151.45 82.975) (end 151.45 85.4) (width 0.2) (layer "F.Cu") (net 16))
 (segment (start 146.8 91.425) (end 150.675 91.425) (width 0.2) (layer "F.Cu") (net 11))
 (segment (start 150.675 91.425) (end 151.4 90.7) (width 0.2) (layer "F.Cu") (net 11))
 (segment (start 146.4 91.025) (end 146.8 91.425) (width 0.2) (layer "F.Cu") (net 11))
 (segment (start 138.955 66.7685) (end 146.4 74.2135) (width 0.2) (layer "F.Cu") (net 11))
 (segment (start 146.4 74.2135) (end 146.4 91.025) (width 0.2) (layer "F.Cu") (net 11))
 (segment (start 86.749999 106.850001) (end 86.749999 69.249999) (width 0.2) (layer "F.Cu") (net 1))
 (segment (start 85.65 107.95) (end 86.749999 106.850001) (width 0.2) (layer "F.Cu") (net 1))
 (segment (start 103.874346 69.2) (end 113.574346 59.5) (width 0.2) (layer "F.Cu") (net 1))
 (segment (start 86.749999 69.249999) (end 86.7 69.2) (width 0.2) (layer "F.Cu") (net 1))
 (segment (start 114.7 59.5) (end 115.0515 59.1485) (width 0.2) (layer "F.Cu") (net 1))
 (segment (start 115.0515 59.1485) (end 122.88 59.1485) (width 0.2) (layer "F.Cu") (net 1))
 (segment (start 113.574346 59.5) (end 114.7 59.5) (width 0.2) (layer "F.Cu") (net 1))
 (segment (start 86.7 69.2) (end 103.874346 69.2) (width 0.2) (layer "F.Cu") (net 1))
 (segment (start 122.88 61.6885) (end 112.943337 61.6885) (width 0.2) (layer "F.Cu") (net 2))
 (segment (start 112.943337 61.6885) (end 104.631837 70) (width 0.2) (layer "F.Cu") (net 2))
 (segment (start 85.65 110.917056) (end 85.65 127.15) (width 0.2) (layer "F.Cu") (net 2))
 (segment (start 87.6 70) (end 87.6 108.967056) (width 0.2) (layer "F.Cu") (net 2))
 (segment (start 87.6 108.967056) (end 85.65 110.917056) (width 0.2) (layer "F.Cu") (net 2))
 (segment (start 104.631837 70) (end 87.6 70) (width 0.2) (layer "F.Cu") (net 2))
 (segment (start 122.88 64.2285) (end 115.211663 64.2285) (width 0.2) (layer "F.Cu") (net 3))
 (segment (start 104.61 74.830163) (end 104.61 107.95) (width 0.2) (layer "F.Cu") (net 3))
 (segment (start 115.211663 64.2285) (end 104.61 74.830163) (width 0.2) (layer "F.Cu") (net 3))
 (segment (start 104.61 110.51) (end 104.61 127.15) (width 0.2) (layer "F.Cu") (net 4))
 (segment (start 113.8315 66.7685) (end 105.01 75.59) (width 0.2) (layer "F.Cu") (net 4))
 (segment (start 105.01 75.59) (end 105.01 105.5) (width 0.2) (layer "F.Cu") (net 4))
 (segment (start 106.01 106.5) (end 106.01 109.09) (width 0.2) (layer "F.Cu") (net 4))
 (segment (start 122.88 66.7685) (end 113.8315 66.7685) (width 0.2) (layer "F.Cu") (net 4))
 (segment (start 105.01 105.5) (end 106.01 106.5) (width 0.2) (layer "F.Cu") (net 4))
 (segment (start 104.6 110.5) (end 104.61 110.51) (width 0.2) (layer "F.Cu") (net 4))
 (segment (start 106.01 109.09) (end 104.6 110.5) (width 0.2) (layer "F.Cu") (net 4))
 (segment (start 135.1 74.8685) (end 138.12 71.8485) (width 0.2) (layer "F.Cu") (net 9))
 (segment (start 129.51 102.1) (end 135.1 102.1) (width 0.2) (layer "F.Cu") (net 9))
 (segment (start 123.65 107.96) (end 129.51 102.1) (width 0.2) (layer "F.Cu") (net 9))
 (segment (start 135.1 102.1) (end 135.1 74.8685) (width 0.2) (layer "F.Cu") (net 9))
 (segment (start 140.471 70.58187) (end 140.471 72.649714) (width 0.2) (layer "F.Cu") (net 10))
 (segment (start 137.623686 72.9105) (end 135.5 75.034186) (width 0.2) (layer "F.Cu") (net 10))
 (segment (start 139.19763 69.3085) (end 140.471 70.58187) (width 0.2) (layer "F.Cu") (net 10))
 (segment (start 140.210214 72.9105) (end 137.623686 72.9105) (width 0.2) (layer "F.Cu") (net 10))
 (segment (start 140.471 72.649714) (end 140.210214 72.9105) (width 0.2) (layer "F.Cu") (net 10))
 (segment (start 138.12 69.3085) (end 139.19763 69.3085) (width 0.2) (layer "F.Cu") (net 10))
 (segment (start 135.5 75.034186) (end 135.5 115.31) (width 0.2) (layer "F.Cu") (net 10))
 (segment (start 135.5 115.31) (end 123.65 127.16) (width 0.2) (layer "F.Cu") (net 10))
 (segment (start 122.88 74.3885) (end 122.118001 75.150499) (width 0.2) (layer "F.Cu") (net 7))
 (segment (start 122.118001 94.118001) (end 129 101) (width 0.2) (layer "F.Cu") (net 7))
 (segment (start 122.118001 75.150499) (end 122.118001 94.118001) (width 0.2) (layer "F.Cu") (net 7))
 (segment (start 139.3 106.7) (end 140.55 107.95) (width 0.2) (layer "F.Cu") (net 7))
 (segment (start 133.2 101) (end 133.3 100.9) (width 0.2) (layer "F.Cu") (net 7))
 (segment (start 140.55 107.95) (end 142.69 107.95) (width 0.2) (layer "F.Cu") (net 7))
 (segment (start 129 101) (end 133.2 101) (width 0.2) (layer "F.Cu") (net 7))
 (via (at 139.3 106.7) (size 0.6) (drill 0.3) (layers "F.Cu" "B.Cu") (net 7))
 (via (at 133.3 100.9) (size 0.6) (drill 0.3) (layers "F.Cu" "B.Cu") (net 7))
 (segment (start 133.3 100.9) (end 139.1 106.7) (width 0.2) (layer "B.Cu") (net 7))
 (segment (start 139.1 106.7) (end 139.3 106.7) (width 0.2) (layer "B.Cu") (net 7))
 (segment (start 144.09 125.75) (end 142.69 127.15) (width 0.2) (layer "F.Cu") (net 8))
 (segment (start 144.09 80.3585) (end 144.09 125.75) (width 0.2) (layer "F.Cu") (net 8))
 (segment (start 138.12 74.3885) (end 144.09 80.3585) (width 0.2) (layer "F.Cu") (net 8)))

